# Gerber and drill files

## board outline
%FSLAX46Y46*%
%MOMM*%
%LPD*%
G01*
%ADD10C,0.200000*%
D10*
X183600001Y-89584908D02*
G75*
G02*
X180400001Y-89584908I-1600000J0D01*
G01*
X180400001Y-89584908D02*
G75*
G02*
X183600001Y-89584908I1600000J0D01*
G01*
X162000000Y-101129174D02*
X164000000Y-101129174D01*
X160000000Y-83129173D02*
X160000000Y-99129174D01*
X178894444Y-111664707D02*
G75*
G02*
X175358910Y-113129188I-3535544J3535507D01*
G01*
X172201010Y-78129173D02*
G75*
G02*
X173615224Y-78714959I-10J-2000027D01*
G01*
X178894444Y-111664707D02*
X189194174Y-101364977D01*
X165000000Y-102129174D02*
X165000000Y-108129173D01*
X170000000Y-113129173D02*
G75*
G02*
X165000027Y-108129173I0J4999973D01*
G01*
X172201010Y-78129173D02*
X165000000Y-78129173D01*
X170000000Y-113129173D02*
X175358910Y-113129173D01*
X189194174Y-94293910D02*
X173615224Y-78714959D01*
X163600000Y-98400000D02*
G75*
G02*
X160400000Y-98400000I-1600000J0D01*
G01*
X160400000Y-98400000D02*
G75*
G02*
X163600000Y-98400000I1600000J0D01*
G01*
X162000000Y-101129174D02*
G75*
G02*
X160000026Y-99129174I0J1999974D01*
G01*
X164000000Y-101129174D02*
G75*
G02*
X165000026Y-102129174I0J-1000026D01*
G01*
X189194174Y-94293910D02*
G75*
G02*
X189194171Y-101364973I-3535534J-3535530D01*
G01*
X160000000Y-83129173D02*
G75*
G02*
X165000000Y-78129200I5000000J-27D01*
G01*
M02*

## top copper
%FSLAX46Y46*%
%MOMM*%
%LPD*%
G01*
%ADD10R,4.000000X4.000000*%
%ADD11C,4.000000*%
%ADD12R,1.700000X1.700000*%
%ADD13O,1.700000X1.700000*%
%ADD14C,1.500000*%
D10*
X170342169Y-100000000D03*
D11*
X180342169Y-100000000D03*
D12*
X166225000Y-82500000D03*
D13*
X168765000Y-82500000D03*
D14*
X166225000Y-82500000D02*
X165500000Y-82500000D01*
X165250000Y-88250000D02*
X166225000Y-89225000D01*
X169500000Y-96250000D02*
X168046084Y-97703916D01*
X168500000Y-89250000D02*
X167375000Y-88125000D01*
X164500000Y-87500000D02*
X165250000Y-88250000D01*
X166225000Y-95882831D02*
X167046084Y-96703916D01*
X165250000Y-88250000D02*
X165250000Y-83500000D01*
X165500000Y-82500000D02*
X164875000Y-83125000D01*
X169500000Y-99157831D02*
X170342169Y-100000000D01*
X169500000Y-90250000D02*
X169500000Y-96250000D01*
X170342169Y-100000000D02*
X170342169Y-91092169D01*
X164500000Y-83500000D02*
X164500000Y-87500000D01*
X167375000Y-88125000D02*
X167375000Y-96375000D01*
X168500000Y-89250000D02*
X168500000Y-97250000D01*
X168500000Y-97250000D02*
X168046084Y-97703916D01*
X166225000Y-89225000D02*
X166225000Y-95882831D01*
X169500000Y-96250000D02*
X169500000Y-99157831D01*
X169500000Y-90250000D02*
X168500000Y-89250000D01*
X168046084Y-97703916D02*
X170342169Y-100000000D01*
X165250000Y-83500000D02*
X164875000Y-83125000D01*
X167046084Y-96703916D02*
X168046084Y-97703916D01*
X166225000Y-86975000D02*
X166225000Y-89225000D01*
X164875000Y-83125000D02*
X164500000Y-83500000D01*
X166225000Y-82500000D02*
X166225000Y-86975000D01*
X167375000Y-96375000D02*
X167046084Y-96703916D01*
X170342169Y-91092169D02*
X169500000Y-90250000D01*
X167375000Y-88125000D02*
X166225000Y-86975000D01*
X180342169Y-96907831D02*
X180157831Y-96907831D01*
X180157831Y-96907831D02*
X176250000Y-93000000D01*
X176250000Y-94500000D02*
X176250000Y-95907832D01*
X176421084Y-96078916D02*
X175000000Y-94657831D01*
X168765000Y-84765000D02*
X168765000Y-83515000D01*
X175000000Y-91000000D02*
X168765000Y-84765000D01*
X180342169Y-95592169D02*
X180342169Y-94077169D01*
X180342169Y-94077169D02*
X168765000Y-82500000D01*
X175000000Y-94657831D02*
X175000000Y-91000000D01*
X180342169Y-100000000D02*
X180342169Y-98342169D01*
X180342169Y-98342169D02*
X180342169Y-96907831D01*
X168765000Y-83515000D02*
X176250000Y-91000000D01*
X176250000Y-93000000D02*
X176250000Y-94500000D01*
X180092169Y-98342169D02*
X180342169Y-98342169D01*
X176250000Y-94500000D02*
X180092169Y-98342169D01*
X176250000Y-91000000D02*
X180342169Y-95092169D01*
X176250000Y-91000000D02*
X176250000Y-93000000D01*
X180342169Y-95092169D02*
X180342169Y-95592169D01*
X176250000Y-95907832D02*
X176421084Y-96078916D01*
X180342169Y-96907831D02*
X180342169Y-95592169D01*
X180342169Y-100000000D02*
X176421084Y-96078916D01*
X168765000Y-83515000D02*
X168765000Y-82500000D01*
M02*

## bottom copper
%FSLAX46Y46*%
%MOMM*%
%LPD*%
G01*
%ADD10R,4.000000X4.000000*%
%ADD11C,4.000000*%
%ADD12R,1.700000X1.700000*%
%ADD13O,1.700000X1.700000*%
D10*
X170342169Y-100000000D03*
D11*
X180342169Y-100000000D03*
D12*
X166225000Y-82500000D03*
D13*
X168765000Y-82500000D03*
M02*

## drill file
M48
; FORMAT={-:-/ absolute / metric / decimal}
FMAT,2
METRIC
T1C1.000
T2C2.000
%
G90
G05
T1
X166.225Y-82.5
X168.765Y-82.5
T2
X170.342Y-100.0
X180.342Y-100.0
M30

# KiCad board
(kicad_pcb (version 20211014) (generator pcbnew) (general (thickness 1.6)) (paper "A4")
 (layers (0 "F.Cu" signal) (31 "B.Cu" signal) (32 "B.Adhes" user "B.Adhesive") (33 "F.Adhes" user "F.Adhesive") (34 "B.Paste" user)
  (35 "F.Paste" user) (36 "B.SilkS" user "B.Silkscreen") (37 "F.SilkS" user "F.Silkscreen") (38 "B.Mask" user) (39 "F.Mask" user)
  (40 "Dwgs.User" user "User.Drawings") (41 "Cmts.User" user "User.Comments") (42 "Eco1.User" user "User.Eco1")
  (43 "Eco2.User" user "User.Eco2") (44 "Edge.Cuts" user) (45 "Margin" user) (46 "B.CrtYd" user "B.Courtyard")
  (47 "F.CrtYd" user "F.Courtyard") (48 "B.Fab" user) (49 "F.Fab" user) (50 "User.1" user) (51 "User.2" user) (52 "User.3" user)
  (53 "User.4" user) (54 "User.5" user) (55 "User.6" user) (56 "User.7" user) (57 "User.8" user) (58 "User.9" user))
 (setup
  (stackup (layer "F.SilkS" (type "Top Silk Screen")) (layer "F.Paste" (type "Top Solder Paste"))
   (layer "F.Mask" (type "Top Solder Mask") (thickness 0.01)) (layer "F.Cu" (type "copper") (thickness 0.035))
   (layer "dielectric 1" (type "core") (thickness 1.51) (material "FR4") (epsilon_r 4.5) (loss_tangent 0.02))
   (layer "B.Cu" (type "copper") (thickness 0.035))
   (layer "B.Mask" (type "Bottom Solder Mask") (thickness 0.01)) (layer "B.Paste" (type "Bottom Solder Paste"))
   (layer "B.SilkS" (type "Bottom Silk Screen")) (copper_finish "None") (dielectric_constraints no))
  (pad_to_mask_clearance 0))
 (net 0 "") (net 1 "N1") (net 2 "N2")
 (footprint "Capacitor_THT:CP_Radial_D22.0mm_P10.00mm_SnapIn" (layer "F.Cu") (at 170.342169 100)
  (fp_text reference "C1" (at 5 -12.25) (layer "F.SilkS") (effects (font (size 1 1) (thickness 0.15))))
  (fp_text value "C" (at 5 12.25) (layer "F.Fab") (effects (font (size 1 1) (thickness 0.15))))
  (pad "1" thru_hole rect (at 0 0) (size 4 4) (drill 2) (layers *.Cu *.Mask) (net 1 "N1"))
  (pad "2" thru_hole circle (at 10 0) (size 4 4) (drill 2) (layers *.Cu *.Mask) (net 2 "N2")))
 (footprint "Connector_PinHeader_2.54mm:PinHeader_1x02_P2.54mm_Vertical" (layer "F.Cu") (at 166.225 82.5 90)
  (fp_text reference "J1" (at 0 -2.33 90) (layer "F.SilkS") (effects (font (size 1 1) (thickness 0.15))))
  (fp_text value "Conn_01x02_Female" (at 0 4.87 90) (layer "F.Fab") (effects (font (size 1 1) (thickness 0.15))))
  (pad "1" thru_hole rect (at 0 0 90) (size 1.7 1.7) (drill 1) (layers *.Cu *.Mask) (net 1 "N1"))
  (pad "2" thru_hole oval (at 0 2.54 90) (size 1.7 1.7) (drill 1) (layers *.Cu *.Mask) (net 2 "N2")))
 (gr_circle (center 182.000001 89.584908) (end 180.400001 89.584908) (layer "Edge.Cuts") (width 0.2) (fill none))
 (gr_line (start 162 101.129174) (end 164 101.129174) (layer "Edge.Cuts") (width 0.2))
 (gr_line (start 160 83.129173) (end 160 99.129174) (layer "Edge.Cuts") (width 0.2))
 (gr_arc (start 178.894444 111.664707) (mid 177.272327 112.748571) (end 175.35891 113.129173) (layer "Edge.Cuts") (width 0.2))
 (gr_arc (start 172.20101 78.129173) (mid 172.966377 78.281414) (end 173.615224 78.714959) (layer "Edge.Cuts") (width 0.2))
 (gr_line (start 178.894444 111.664707) (end 189.194174 101.364977) (layer "Edge.Cuts") (width 0.2))
 (gr_line (start 165 102.129174) (end 165 108.129173) (layer "Edge.Cuts") (width 0.2))
 (gr_arc (start 170 113.129173) (mid 166.464466 111.664707) (end 165 108.129173) (layer "Edge.Cuts") (width 0.2))
 (gr_line (start 172.20101 78.129173) (end 165 78.129173) (layer "Edge.Cuts") (width 0.2))
 (gr_line (start 170 113.129173) (end 175.35891 113.129173) (layer "Edge.Cuts") (width 0.2))
 (gr_line (start 189.194174 94.29391) (end 173.615224 78.714959) (layer "Edge.Cuts") (width 0.2))
 (gr_circle (center 162 98.4) (end 160.4 98.4) (layer "Edge.Cuts") (width 0.2) (fill none))
 (gr_arc (start 162 101.129174) (mid 160.585786 100.543388) (end 160 99.129174) (layer "Edge.Cuts") (width 0.2))
 (gr_arc (start 164 101.129174) (mid 164.707107 101.422067) (end 165 102.129174) (layer "Edge.Cuts") (width 0.2))
 (gr_arc (start 189.194174 94.29391) (mid 190.65864 97.829444) (end 189.194174 101.364977) (layer "Edge.Cuts") (width 0.2))
 (gr_arc (start 160 83.129173) (mid 161.464466 79.593639) (end 165 78.129173) (layer "Edge.Cuts") (width 0.2))
 (segment (start 166.225 82.5) (end 165.5 82.5) (width 1.5) (layer "F.Cu") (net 1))
 (segment (start 165.25 88.25) (end 166.225 89.225) (width 1.5) (layer "F.Cu") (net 1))
 (segment (start 169.5 96.25) (end 168.046084 97.703916) (width 1.5) (layer "F.Cu") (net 1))
 (segment (start 168.5 89.25) (end 167.375 88.125) (width 1.5) (layer "F.Cu") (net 1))
 (segment (start 164.5 87.5) (end 165.25 88.25) (width 1.5) (layer "F.Cu") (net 1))
 (segment (start 166.225 95.882831) (end 167.046084 96.703916) (width 1.5) (layer "F.Cu") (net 1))
 (segment (start 165.25 88.25) (end 165.25 83.5) (width 1.5) (layer "F.Cu") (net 1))
 (segment (start 165.5 82.5) (end 164.875 83.125) (width 1.5) (layer "F.Cu") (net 1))
 (segment (start 169.5 99.157831) (end 170.342169 100) (width 1.5) (layer "F.Cu") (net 1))
 (segment (start 169.5 90.25) (end 169.5 96.25) (width 1.5) (layer "F.Cu") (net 1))
 (segment (start 170.342169 100) (end 170.342169 91.092169) (width 1.5) (layer "F.Cu") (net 1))
 (segment (start 164.5 83.5) (end 164.5 87.5) (width 1.5) (layer "F.Cu") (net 1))
 (segment (start 167.375 88.125) (end 167.375 96.375) (width 1.5) (layer "F.Cu") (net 1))
 (segment (start 168.5 89.25) (end 168.5 97.25) (width 1.5) (layer "F.Cu") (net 1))
 (segment (start 168.5 97.25) (end 168.046084 97.703916) (width 1.5) (layer "F.Cu") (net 1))
 (segment (start 166.225 89.225) (end 166.225 95.882831) (width 1.5) (layer "F.Cu") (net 1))
 (segment (start 169.5 96.25) (end 169.5 99.157831) (width 1.5) (layer "F.Cu") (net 1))
 (segment (start 169.5 90.25) (end 168.5 89.25) (width 1.5) (layer "F.Cu") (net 1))
 (segment (start 168.046084 97.703916) (end 170.342169 100) (width 1.5) (layer "F.Cu") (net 1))
 (segment (start 165.25 83.5) (end 164.875 83.125) (width 1.5) (layer "F.Cu") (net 1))
 (segment (start 167.046084 96.703916) (end 168.046084 97.703916) (width 1.5) (layer "F.Cu") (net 1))
 (segment (start 166.225 86.975) (end 166.225 89.225) (width 1.5) (layer "F.Cu") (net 1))
 (segment (start 164.875 83.125) (end 164.5 83.5) (width 1.5) (layer "F.Cu") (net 1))
 (segment (start 166.225 82.5) (end 166.225 86.975) (width 1.5) (layer "F.Cu") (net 1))
 (segment (start 167.375 96.375) (end 167.046084 96.703916) (width 1.5) (layer "F.Cu") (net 1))
 (segment (start 170.342169 91.092169) (end 169.5 90.25) (width 1.5) (layer "F.Cu") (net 1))
 (segment (start 167.375 88.125) (end 166.225 86.975) (width 1.5) (layer "F.Cu") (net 1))
 (segment (start 180.342169 96.907831) (end 180.157831 96.907831) (width 1.5) (layer "F.Cu") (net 2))
 (segment (start 180.157831 96.907831) (end 176.25 93) (width 1.5) (layer "F.Cu") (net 2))
 (segment (start 176.25 94.5) (end 176.25 95.907832) (width 1.5) (layer "F.Cu") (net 2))
 (segment (start 176.421084 96.078916) (end 175 94.657831) (width 1.5) (layer "F.Cu") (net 2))
 (segment (start 168.765 84.765) (end 168.765 83.515) (width 1.5) (layer "F.Cu") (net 2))
 (segment (start 175 91) (end 168.765 84.765) (width 1.5) (layer "F.Cu") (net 2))
 (segment (start 180.342169 95.592169) (end 180.342169 94.077169) (width 1.5) (layer "F.Cu") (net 2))
 (segment (start 180.342169 94.077169) (end 168.765 82.5) (width 1.5) (layer "F.Cu") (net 2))
 (segment (start 175 94.657831) (end 175 91) (width 1.5) (layer "F.Cu") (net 2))
 (segment (start 180.342169 100) (end 180.342169 98.342169) (width 1.5) (layer "F.Cu") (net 2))
 (segment (start 180.342169 98.342169) (end 180.342169 96.907831) (width 1.5) (layer "F.Cu") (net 2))
 (segment (start 168.765 83.515) (end 176.25 91) (width 1.5) (layer "F.Cu") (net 2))
 (segment (start 176.25 93) (end 176.25 94.5) (width 1.5) (layer "F.Cu") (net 2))
 (segment (start 180.092169 98.342169) (end 180.342169 98.342169) (width 1.5) (layer "F.Cu") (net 2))
 (segment (start 176.25 94.5) (end 180.092169 98.342169) (width 1.5) (layer "F.Cu") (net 2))
 (segment (start 176.25 91) (end 180.342169 95.092169) (width 1.5) (layer "F.Cu") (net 2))
 (segment (start 176.25 91) (end 176.25 93) (width 1.5) (layer "F.Cu") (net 2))
 (segment (start 180.342169 95.092169) (end 180.342169 95.592169) (width 1.5) (layer "F.Cu") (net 2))
 (segment (start 176.25 95.907832) (end 176.421084 96.078916) (width 1.5) (layer "F.Cu") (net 2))
 (segment (start 180.342169 96.907831) (end 180.342169 95.592169) (width 1.5) (layer "F.Cu") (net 2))
 (segment (start 180.342169 100) (end 176.421084 96.078916) (width 1.5) (layer "F.Cu") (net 2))
 (segment (start 168.765 83.515) (end 168.765 82.5) (width 1.5) (layer "F.Cu") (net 2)))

